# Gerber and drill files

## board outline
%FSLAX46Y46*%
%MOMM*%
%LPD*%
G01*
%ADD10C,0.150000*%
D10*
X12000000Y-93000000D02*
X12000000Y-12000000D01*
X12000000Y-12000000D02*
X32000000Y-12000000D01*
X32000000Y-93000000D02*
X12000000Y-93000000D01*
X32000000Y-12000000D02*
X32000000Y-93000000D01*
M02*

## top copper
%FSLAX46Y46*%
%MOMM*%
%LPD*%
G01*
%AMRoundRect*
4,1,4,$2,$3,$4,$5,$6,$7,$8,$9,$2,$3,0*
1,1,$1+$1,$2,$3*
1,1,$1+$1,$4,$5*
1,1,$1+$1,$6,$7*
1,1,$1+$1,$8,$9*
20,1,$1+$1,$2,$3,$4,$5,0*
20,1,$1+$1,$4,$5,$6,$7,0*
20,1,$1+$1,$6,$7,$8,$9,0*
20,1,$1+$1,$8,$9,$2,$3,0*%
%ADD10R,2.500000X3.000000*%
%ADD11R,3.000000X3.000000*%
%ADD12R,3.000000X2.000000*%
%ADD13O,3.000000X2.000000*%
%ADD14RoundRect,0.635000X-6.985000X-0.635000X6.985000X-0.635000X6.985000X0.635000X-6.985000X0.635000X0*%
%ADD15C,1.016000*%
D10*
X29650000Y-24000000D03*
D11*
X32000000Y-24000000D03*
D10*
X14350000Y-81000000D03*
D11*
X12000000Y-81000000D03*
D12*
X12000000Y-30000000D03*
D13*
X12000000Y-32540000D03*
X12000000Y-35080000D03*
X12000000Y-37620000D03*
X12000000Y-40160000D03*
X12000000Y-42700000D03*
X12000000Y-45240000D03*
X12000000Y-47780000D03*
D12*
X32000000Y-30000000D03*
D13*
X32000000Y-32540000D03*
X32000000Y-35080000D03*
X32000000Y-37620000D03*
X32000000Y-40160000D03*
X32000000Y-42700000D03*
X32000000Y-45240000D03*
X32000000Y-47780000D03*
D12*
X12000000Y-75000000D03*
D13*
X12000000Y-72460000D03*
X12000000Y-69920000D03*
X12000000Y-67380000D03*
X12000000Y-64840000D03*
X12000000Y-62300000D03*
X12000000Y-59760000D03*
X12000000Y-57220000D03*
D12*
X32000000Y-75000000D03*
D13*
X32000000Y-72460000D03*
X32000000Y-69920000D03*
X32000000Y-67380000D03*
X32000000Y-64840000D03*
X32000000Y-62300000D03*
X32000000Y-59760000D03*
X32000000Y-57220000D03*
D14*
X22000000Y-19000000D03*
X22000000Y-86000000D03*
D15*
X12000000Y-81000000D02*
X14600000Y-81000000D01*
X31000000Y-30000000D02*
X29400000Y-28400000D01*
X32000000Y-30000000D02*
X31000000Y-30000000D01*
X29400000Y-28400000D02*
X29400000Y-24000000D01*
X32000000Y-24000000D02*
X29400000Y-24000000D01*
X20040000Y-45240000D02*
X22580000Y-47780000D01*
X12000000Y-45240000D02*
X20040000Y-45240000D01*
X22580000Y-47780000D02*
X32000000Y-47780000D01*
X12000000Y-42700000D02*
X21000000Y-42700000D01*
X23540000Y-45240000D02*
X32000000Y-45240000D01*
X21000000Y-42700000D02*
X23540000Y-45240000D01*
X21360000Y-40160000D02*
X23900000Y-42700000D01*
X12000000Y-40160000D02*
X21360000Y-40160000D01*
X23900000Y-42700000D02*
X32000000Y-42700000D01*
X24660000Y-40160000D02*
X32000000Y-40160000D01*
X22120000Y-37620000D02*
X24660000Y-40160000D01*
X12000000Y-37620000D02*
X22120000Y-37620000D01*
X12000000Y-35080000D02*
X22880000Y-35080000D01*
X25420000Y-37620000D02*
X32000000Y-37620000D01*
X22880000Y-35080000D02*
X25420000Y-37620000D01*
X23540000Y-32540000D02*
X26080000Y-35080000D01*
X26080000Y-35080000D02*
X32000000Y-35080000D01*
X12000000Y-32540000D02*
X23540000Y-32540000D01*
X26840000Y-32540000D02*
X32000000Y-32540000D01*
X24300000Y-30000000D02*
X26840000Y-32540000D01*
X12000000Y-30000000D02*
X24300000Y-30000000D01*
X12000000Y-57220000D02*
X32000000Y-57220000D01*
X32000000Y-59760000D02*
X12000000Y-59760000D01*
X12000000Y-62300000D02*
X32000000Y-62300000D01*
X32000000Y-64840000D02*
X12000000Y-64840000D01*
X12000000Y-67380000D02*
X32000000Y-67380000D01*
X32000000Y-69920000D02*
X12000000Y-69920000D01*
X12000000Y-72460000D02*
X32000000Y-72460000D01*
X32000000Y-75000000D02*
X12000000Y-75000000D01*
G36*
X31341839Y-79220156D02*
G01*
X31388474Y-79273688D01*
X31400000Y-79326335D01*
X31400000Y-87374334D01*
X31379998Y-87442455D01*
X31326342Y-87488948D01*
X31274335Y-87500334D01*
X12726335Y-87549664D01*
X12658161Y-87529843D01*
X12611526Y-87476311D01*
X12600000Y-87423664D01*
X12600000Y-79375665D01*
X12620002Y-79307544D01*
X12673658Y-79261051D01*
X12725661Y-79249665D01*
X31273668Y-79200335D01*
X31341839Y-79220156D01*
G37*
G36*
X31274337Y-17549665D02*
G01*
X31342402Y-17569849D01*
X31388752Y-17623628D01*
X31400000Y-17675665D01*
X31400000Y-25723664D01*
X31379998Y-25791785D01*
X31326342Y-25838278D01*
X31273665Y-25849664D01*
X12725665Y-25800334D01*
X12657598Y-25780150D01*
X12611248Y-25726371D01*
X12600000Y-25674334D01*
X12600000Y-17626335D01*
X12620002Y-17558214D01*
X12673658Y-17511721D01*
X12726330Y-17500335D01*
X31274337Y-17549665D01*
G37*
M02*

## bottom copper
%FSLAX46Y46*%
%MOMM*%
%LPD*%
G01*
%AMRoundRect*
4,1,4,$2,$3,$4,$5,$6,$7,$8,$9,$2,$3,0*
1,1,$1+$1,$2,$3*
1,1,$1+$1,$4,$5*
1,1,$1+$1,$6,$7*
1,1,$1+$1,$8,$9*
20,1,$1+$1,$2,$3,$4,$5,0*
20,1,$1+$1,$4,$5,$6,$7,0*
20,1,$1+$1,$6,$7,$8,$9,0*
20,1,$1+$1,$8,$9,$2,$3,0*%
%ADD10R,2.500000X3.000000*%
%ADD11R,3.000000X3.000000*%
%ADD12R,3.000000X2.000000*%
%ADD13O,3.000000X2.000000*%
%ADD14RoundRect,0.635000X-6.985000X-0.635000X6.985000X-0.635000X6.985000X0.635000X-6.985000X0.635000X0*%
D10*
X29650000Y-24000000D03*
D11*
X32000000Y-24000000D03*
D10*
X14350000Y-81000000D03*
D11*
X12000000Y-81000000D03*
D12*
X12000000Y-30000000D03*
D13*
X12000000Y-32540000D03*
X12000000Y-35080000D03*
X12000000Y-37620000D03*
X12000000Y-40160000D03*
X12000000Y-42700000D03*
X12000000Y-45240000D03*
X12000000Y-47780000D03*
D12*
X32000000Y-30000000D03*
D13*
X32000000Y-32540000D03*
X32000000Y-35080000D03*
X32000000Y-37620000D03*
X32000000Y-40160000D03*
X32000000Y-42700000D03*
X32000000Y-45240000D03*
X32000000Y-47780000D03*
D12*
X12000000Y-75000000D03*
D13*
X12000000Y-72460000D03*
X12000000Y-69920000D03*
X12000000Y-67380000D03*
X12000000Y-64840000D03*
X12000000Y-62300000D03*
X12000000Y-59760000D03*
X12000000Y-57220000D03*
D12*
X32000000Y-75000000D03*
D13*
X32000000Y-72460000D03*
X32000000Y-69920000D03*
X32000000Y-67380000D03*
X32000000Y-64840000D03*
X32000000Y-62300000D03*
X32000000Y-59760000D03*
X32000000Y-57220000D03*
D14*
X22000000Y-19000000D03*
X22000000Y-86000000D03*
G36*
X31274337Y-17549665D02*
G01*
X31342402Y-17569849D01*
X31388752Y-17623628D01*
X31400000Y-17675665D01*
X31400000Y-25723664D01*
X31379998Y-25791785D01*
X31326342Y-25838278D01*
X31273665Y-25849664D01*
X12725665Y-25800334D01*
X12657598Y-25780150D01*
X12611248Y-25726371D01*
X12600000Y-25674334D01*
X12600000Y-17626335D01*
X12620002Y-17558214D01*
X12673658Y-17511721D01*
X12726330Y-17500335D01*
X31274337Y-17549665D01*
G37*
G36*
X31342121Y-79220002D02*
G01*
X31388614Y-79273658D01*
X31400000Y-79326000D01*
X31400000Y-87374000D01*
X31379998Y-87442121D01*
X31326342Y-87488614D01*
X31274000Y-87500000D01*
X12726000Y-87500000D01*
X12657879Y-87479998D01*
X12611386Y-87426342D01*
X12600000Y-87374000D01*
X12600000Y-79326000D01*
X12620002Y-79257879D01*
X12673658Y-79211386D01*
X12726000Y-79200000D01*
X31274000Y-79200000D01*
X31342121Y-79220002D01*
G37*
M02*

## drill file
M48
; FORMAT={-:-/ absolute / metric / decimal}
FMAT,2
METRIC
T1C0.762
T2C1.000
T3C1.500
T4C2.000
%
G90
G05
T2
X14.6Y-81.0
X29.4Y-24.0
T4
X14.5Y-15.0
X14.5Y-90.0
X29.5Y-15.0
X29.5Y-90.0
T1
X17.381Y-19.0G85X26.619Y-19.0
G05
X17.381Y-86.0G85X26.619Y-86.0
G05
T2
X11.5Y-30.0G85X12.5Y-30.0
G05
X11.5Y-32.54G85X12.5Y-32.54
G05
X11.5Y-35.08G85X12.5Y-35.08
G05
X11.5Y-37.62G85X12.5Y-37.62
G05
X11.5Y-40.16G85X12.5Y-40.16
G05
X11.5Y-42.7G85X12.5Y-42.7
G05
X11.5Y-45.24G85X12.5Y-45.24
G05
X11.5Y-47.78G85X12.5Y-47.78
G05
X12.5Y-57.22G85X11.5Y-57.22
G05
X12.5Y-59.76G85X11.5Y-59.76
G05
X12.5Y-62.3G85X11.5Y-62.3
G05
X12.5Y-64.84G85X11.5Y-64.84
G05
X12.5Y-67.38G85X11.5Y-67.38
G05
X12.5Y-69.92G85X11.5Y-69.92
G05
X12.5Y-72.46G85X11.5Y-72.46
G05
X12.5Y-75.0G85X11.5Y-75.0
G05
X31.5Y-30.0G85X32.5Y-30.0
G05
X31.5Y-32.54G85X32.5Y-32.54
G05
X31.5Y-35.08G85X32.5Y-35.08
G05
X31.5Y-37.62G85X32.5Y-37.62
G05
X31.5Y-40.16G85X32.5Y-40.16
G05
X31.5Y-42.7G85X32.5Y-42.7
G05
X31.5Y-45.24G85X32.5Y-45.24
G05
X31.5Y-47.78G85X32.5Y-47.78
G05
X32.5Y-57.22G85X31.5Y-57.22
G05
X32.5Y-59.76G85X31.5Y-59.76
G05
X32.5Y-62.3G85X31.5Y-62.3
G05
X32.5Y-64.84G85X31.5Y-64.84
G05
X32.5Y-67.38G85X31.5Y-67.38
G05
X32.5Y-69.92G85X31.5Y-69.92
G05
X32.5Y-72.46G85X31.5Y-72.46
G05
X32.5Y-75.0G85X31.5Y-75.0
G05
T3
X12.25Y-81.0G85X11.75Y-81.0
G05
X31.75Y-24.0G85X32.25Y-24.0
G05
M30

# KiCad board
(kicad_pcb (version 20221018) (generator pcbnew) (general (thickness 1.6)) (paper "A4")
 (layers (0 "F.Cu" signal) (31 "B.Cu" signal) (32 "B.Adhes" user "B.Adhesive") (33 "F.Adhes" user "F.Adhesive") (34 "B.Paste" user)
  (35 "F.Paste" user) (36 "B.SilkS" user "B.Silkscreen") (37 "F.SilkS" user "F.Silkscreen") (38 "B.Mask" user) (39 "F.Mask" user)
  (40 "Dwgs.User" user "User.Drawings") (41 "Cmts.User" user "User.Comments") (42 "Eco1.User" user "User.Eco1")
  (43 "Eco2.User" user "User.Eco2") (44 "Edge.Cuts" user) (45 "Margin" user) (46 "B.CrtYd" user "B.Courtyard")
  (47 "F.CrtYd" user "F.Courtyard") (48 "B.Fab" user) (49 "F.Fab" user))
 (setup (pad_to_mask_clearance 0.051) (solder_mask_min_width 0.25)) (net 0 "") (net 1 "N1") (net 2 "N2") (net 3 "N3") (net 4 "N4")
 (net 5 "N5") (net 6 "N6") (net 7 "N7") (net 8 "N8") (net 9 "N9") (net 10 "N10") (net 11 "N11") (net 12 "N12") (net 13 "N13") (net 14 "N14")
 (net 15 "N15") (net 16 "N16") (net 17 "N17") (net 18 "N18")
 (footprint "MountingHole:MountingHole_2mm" (layer "F.Cu") (at 14.5 15)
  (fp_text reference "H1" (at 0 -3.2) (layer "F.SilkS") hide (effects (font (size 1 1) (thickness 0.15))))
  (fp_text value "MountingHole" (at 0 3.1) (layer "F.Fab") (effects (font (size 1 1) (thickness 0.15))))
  (pad "" np_thru_hole circle (at 0 0) (size 2 2) (drill 2) (layers "*.Cu" "*.Mask")))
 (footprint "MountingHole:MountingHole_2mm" (layer "F.Cu") (at 29.5 15)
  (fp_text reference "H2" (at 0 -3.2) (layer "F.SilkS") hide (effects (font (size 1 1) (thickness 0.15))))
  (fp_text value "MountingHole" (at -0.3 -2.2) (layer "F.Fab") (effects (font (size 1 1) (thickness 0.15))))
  (pad "" np_thru_hole circle (at 0 0) (size 2 2) (drill 2) (layers "*.Cu" "*.Mask")))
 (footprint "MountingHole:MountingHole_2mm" (layer "F.Cu") (at 29.5 90)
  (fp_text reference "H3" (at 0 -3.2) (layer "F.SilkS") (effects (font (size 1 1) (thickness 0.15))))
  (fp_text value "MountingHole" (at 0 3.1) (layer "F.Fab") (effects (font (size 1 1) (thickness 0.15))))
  (pad "" np_thru_hole circle (at 0 0) (size 2 2) (drill 2) (layers "*.Cu" "*.Mask")))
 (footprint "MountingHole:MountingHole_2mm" (layer "F.Cu") (at 14.5 90)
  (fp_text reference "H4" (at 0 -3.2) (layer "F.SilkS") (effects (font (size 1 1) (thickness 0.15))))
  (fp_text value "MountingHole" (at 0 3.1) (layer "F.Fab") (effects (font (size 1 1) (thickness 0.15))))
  (pad "" np_thru_hole circle (at 0 0) (size 2 2) (drill 2) (layers "*.Cu" "*.Mask")))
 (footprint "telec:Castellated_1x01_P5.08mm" (layer "F.Cu") (at 32 24)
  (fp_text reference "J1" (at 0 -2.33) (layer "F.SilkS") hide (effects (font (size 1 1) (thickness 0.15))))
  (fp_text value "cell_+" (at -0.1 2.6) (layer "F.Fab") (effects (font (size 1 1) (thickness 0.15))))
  (pad "1" thru_hole rect (at -2.6 0) (size 2.5 3) (drill 1 (offset 0.25 0)) (layers "*.Cu" "*.Mask") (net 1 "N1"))
  (pad "1" thru_hole rect (at 0 0) (size 3 3) (drill oval 2 1.5) (layers "*.Cu" "*.Mask") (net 1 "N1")))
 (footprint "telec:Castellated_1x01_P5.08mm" (layer "F.Cu") (at 12 81 180)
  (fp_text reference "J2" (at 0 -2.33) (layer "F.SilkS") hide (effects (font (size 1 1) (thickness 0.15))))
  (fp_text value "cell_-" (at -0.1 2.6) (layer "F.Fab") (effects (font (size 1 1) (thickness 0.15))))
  (pad "1" thru_hole rect (at -2.6 0 180) (size 2.5 3) (drill 1 (offset 0.25 0)) (layers "*.Cu" "*.Mask") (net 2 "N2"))
  (pad "1" thru_hole rect (at 0 0 180) (size 3 3) (drill oval 2 1.5) (layers "*.Cu" "*.Mask") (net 2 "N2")))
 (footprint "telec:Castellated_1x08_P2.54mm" (layer "F.Cu") (at 12 30)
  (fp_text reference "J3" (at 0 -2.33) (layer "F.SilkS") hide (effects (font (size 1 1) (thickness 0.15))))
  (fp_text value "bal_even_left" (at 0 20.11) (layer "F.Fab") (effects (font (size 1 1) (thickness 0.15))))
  (pad "1" thru_hole rect (at 0 0) (size 3 2) (drill oval 2 1) (layers "*.Cu" "*.Mask") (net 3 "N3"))
  (pad "2" thru_hole oval (at 0 2.54) (size 3 2) (drill oval 2 1) (layers "*.Cu" "*.Mask") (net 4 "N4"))
  (pad "3" thru_hole oval (at 0 5.08) (size 3 2) (drill oval 2 1) (layers "*.Cu" "*.Mask") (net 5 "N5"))
  (pad "4" thru_hole oval (at 0 7.62) (size 3 2) (drill oval 2 1) (layers "*.Cu" "*.Mask") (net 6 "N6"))
  (pad "5" thru_hole oval (at 0 10.16) (size 3 2) (drill oval 2 1) (layers "*.Cu" "*.Mask") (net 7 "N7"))
  (pad "6" thru_hole oval (at 0 12.7) (size 3 2) (drill oval 2 1) (layers "*.Cu" "*.Mask") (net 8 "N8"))
  (pad "7" thru_hole oval (at 0 15.24) (size 3 2) (drill oval 2 1) (layers "*.Cu" "*.Mask") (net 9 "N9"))
  (pad "8" thru_hole oval (at 0 17.78) (size 3 2) (drill oval 2 1) (layers "*.Cu" "*.Mask") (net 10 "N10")))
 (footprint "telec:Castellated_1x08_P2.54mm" (layer "F.Cu") (at 32 30)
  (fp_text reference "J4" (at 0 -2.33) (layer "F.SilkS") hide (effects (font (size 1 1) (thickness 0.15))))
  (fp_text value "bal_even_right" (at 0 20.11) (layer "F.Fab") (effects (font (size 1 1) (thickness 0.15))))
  (pad "1" thru_hole rect (at 0 0) (size 3 2) (drill oval 2 1) (layers "*.Cu" "*.Mask") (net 1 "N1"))
  (pad "2" thru_hole oval (at 0 2.54) (size 3 2) (drill oval 2 1) (layers "*.Cu" "*.Mask") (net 3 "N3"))
  (pad "3" thru_hole oval (at 0 5.08) (size 3 2) (drill oval 2 1) (layers "*.Cu" "*.Mask") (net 4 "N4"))
  (pad "4" thru_hole oval (at 0 7.62) (size 3 2) (drill oval 2 1) (layers "*.Cu" "*.Mask") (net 5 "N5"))
  (pad "5" thru_hole oval (at 0 10.16) (size 3 2) (drill oval 2 1) (layers "*.Cu" "*.Mask") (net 6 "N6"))
  (pad "6" thru_hole oval (at 0 12.7) (size 3 2) (drill oval 2 1) (layers "*.Cu" "*.Mask") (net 7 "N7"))
  (pad "7" thru_hole oval (at 0 15.24) (size 3 2) (drill oval 2 1) (layers "*.Cu" "*.Mask") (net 8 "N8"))
  (pad "8" thru_hole oval (at 0 17.78) (size 3 2) (drill oval 2 1) (layers "*.Cu" "*.Mask") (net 9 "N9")))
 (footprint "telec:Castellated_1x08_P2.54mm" (layer "F.Cu") (at 12 75 180)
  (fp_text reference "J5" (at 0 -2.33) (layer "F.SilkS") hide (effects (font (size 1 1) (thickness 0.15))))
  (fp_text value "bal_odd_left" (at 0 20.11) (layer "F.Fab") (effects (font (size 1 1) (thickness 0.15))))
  (pad "1" thru_hole rect (at 0 0 180) (size 3 2) (drill oval 2 1) (layers "*.Cu" "*.Mask") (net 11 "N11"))
  (pad "2" thru_hole oval (at 0 2.54 180) (size 3 2) (drill oval 2 1) (layers "*.Cu" "*.Mask") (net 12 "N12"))
  (pad "3" thru_hole oval (at 0 5.08 180) (size 3 2) (drill oval 2 1) (layers "*.Cu" "*.Mask") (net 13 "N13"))
  (pad "4" thru_hole oval (at 0 7.62 180) (size 3 2) (drill oval 2 1) (layers "*.Cu" "*.Mask") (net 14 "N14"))
  (pad "5" thru_hole oval (at 0 10.16 180) (size 3 2) (drill oval 2 1) (layers "*.Cu" "*.Mask") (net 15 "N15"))
  (pad "6" thru_hole oval (at 0 12.7 180) (size 3 2) (drill oval 2 1) (layers "*.Cu" "*.Mask") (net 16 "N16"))
  (pad "7" thru_hole oval (at 0 15.24 180) (size 3 2) (drill oval 2 1) (layers "*.Cu" "*.Mask") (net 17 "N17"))
  (pad "8" thru_hole oval (at 0 17.78 180) (size 3 2) (drill oval 2 1) (layers "*.Cu" "*.Mask") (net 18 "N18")))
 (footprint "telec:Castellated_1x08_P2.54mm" (layer "F.Cu") (at 32 75 180)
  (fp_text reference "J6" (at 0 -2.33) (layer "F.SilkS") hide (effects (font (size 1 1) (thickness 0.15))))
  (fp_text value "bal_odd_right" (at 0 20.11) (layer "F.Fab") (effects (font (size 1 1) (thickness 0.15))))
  (pad "1" thru_hole rect (at 0 0 180) (size 3 2) (drill oval 2 1) (layers "*.Cu" "*.Mask") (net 11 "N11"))
  (pad "2" thru_hole oval (at 0 2.54 180) (size 3 2) (drill oval 2 1) (layers "*.Cu" "*.Mask") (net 12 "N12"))
  (pad "3" thru_hole oval (at 0 5.08 180) (size 3 2) (drill oval 2 1) (layers "*.Cu" "*.Mask") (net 13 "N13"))
  (pad "4" thru_hole oval (at 0 7.62 180) (size 3 2) (drill oval 2 1) (layers "*.Cu" "*.Mask") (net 14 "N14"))
  (pad "5" thru_hole oval (at 0 10.16 180) (size 3 2) (drill oval 2 1) (layers "*.Cu" "*.Mask") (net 15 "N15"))
  (pad "6" thru_hole oval (at 0 12.7 180) (size 3 2) (drill oval 2 1) (layers "*.Cu" "*.Mask") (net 16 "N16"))
  (pad "7" thru_hole oval (at 0 15.24 180) (size 3 2) (drill oval 2 1) (layers "*.Cu" "*.Mask") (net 17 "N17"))
  (pad "8" thru_hole oval (at 0 17.78 180) (size 3 2) (drill oval 2 1) (layers "*.Cu" "*.Mask") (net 18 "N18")))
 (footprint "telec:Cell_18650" (layer "F.Cu") (at 22 19)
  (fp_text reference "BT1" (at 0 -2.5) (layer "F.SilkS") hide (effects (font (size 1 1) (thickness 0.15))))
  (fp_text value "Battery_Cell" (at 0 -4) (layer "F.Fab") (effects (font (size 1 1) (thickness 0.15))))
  (pad "1" thru_hole roundrect (at 0 0) (size 15.24 2.54) (drill oval 10 0.762) (layers "*.Cu" "*.Mask") (roundrect_rratio 0.25)
   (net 1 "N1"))
  (pad "2" thru_hole roundrect (at 0 67) (size 15.24 2.54) (drill oval 10 0.762) (layers "*.Cu" "*.Mask") (roundrect_rratio 0.25)
   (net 2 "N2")))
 (gr_line (start 12 93) (end 12 12) (stroke (width 0.15) (type solid)) (layer "Edge.Cuts"))
 (gr_line (start 12 12) (end 32 12) (stroke (width 0.15) (type solid)) (layer "Edge.Cuts"))
 (gr_line (start 32 93) (end 12 93) (stroke (width 0.15) (type solid)) (layer "Edge.Cuts"))
 (gr_line (start 32 12) (end 32 93) (stroke (width 0.15) (type solid)) (layer "Edge.Cuts"))
 (segment (start 12 81) (end 14.6 81) (width 1.016) (layer "F.Cu") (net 2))
 (segment (start 31 30) (end 29.4 28.4) (width 1.016) (layer "F.Cu") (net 1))
 (segment (start 32 30) (end 31 30) (width 1.016) (layer "F.Cu") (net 1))
 (segment (start 29.4 28.4) (end 29.4 24) (width 1.016) (layer "F.Cu") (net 1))
 (segment (start 32 24) (end 29.4 24) (width 1.016) (layer "F.Cu") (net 1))
 (segment (start 20.04 45.24) (end 22.58 47.78) (width 1.016) (layer "F.Cu") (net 9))
 (segment (start 12 45.24) (end 20.04 45.24) (width 1.016) (layer "F.Cu") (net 9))
 (segment (start 22.58 47.78) (end 32 47.78) (width 1.016) (layer "F.Cu") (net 9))
 (segment (start 12 42.7) (end 21 42.7) (width 1.016) (layer "F.Cu") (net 8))
 (segment (start 23.54 45.24) (end 32 45.24) (width 1.016) (layer "F.Cu") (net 8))
 (segment (start 21 42.7) (end 23.54 45.24) (width 1.016) (layer "F.Cu") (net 8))
 (segment (start 21.36 40.16) (end 23.9 42.7) (width 1.016) (layer "F.Cu") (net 7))
 (segment (start 12 40.16) (end 21.36 40.16) (width 1.016) (layer "F.Cu") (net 7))
 (segment (start 23.9 42.7) (end 32 42.7) (width 1.016) (layer "F.Cu") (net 7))
 (segment (start 24.66 40.16) (end 32 40.16) (width 1.016) (layer "F.Cu") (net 6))
 (segment (start 22.12 37.62) (end 24.66 40.16) (width 1.016) (layer "F.Cu") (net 6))
 (segment (start 12 37.62) (end 22.12 37.62) (width 1.016) (layer "F.Cu") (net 6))
 (segment (start 12 35.08) (end 22.88 35.08) (width 1.016) (layer "F.Cu") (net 5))
 (segment (start 25.42 37.62) (end 32 37.62) (width 1.016) (layer "F.Cu") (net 5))
 (segment (start 22.88 35.08) (end 25.42 37.62) (width 1.016) (layer "F.Cu") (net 5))
 (segment (start 23.54 32.54) (end 26.08 35.08) (width 1.016) (layer "F.Cu") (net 4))
 (segment (start 26.08 35.08) (end 32 35.08) (width 1.016) (layer "F.Cu") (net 4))
 (segment (start 12 32.54) (end 23.54 32.54) (width 1.016) (layer "F.Cu") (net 4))
 (segment (start 26.84 32.54) (end 32 32.54) (width 1.016) (layer "F.Cu") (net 3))
 (segment (start 24.3 30) (end 26.84 32.54) (width 1.016) (layer "F.Cu") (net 3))
 (segment (start 12 30) (end 24.3 30) (width 1.016) (layer "F.Cu") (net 3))
 (segment (start 12 57.22) (end 32 57.22) (width 1.016) (layer "F.Cu") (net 18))
 (segment (start 32 59.76) (end 12 59.76) (width 1.016) (layer "F.Cu") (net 17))
 (segment (start 12 62.3) (end 32 62.3) (width 1.016) (layer "F.Cu") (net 16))
 (segment (start 32 64.84) (end 12 64.84) (width 1.016) (layer "F.Cu") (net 15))
 (segment (start 12 67.38) (end 32 67.38) (width 1.016) (layer "F.Cu") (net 14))
 (segment (start 32 69.92) (end 12 69.92) (width 1.016) (layer "F.Cu") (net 13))
 (segment (start 12 72.46) (end 32 72.46) (width 1.016) (layer "F.Cu") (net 12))
 (segment (start 32 75) (end 12 75) (width 1.016) (layer "F.Cu") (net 11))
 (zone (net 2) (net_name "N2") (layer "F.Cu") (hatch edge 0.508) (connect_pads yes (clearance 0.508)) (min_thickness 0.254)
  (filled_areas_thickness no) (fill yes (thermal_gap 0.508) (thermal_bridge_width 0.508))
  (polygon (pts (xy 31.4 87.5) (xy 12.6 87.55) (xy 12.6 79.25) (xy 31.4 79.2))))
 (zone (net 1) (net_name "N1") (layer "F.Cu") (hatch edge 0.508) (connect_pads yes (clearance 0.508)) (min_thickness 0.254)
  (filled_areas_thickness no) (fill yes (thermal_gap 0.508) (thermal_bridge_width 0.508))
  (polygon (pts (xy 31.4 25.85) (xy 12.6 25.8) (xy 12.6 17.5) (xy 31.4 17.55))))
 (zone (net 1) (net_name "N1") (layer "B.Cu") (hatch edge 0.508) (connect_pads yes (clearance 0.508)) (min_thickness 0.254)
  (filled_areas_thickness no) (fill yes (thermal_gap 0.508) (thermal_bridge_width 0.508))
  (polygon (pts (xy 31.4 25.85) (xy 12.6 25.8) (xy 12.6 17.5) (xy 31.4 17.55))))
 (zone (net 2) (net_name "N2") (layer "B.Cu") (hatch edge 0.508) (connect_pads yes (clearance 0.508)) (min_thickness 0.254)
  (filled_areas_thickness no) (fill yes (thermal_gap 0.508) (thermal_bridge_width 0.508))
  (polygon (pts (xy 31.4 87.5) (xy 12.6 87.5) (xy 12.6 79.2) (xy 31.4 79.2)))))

